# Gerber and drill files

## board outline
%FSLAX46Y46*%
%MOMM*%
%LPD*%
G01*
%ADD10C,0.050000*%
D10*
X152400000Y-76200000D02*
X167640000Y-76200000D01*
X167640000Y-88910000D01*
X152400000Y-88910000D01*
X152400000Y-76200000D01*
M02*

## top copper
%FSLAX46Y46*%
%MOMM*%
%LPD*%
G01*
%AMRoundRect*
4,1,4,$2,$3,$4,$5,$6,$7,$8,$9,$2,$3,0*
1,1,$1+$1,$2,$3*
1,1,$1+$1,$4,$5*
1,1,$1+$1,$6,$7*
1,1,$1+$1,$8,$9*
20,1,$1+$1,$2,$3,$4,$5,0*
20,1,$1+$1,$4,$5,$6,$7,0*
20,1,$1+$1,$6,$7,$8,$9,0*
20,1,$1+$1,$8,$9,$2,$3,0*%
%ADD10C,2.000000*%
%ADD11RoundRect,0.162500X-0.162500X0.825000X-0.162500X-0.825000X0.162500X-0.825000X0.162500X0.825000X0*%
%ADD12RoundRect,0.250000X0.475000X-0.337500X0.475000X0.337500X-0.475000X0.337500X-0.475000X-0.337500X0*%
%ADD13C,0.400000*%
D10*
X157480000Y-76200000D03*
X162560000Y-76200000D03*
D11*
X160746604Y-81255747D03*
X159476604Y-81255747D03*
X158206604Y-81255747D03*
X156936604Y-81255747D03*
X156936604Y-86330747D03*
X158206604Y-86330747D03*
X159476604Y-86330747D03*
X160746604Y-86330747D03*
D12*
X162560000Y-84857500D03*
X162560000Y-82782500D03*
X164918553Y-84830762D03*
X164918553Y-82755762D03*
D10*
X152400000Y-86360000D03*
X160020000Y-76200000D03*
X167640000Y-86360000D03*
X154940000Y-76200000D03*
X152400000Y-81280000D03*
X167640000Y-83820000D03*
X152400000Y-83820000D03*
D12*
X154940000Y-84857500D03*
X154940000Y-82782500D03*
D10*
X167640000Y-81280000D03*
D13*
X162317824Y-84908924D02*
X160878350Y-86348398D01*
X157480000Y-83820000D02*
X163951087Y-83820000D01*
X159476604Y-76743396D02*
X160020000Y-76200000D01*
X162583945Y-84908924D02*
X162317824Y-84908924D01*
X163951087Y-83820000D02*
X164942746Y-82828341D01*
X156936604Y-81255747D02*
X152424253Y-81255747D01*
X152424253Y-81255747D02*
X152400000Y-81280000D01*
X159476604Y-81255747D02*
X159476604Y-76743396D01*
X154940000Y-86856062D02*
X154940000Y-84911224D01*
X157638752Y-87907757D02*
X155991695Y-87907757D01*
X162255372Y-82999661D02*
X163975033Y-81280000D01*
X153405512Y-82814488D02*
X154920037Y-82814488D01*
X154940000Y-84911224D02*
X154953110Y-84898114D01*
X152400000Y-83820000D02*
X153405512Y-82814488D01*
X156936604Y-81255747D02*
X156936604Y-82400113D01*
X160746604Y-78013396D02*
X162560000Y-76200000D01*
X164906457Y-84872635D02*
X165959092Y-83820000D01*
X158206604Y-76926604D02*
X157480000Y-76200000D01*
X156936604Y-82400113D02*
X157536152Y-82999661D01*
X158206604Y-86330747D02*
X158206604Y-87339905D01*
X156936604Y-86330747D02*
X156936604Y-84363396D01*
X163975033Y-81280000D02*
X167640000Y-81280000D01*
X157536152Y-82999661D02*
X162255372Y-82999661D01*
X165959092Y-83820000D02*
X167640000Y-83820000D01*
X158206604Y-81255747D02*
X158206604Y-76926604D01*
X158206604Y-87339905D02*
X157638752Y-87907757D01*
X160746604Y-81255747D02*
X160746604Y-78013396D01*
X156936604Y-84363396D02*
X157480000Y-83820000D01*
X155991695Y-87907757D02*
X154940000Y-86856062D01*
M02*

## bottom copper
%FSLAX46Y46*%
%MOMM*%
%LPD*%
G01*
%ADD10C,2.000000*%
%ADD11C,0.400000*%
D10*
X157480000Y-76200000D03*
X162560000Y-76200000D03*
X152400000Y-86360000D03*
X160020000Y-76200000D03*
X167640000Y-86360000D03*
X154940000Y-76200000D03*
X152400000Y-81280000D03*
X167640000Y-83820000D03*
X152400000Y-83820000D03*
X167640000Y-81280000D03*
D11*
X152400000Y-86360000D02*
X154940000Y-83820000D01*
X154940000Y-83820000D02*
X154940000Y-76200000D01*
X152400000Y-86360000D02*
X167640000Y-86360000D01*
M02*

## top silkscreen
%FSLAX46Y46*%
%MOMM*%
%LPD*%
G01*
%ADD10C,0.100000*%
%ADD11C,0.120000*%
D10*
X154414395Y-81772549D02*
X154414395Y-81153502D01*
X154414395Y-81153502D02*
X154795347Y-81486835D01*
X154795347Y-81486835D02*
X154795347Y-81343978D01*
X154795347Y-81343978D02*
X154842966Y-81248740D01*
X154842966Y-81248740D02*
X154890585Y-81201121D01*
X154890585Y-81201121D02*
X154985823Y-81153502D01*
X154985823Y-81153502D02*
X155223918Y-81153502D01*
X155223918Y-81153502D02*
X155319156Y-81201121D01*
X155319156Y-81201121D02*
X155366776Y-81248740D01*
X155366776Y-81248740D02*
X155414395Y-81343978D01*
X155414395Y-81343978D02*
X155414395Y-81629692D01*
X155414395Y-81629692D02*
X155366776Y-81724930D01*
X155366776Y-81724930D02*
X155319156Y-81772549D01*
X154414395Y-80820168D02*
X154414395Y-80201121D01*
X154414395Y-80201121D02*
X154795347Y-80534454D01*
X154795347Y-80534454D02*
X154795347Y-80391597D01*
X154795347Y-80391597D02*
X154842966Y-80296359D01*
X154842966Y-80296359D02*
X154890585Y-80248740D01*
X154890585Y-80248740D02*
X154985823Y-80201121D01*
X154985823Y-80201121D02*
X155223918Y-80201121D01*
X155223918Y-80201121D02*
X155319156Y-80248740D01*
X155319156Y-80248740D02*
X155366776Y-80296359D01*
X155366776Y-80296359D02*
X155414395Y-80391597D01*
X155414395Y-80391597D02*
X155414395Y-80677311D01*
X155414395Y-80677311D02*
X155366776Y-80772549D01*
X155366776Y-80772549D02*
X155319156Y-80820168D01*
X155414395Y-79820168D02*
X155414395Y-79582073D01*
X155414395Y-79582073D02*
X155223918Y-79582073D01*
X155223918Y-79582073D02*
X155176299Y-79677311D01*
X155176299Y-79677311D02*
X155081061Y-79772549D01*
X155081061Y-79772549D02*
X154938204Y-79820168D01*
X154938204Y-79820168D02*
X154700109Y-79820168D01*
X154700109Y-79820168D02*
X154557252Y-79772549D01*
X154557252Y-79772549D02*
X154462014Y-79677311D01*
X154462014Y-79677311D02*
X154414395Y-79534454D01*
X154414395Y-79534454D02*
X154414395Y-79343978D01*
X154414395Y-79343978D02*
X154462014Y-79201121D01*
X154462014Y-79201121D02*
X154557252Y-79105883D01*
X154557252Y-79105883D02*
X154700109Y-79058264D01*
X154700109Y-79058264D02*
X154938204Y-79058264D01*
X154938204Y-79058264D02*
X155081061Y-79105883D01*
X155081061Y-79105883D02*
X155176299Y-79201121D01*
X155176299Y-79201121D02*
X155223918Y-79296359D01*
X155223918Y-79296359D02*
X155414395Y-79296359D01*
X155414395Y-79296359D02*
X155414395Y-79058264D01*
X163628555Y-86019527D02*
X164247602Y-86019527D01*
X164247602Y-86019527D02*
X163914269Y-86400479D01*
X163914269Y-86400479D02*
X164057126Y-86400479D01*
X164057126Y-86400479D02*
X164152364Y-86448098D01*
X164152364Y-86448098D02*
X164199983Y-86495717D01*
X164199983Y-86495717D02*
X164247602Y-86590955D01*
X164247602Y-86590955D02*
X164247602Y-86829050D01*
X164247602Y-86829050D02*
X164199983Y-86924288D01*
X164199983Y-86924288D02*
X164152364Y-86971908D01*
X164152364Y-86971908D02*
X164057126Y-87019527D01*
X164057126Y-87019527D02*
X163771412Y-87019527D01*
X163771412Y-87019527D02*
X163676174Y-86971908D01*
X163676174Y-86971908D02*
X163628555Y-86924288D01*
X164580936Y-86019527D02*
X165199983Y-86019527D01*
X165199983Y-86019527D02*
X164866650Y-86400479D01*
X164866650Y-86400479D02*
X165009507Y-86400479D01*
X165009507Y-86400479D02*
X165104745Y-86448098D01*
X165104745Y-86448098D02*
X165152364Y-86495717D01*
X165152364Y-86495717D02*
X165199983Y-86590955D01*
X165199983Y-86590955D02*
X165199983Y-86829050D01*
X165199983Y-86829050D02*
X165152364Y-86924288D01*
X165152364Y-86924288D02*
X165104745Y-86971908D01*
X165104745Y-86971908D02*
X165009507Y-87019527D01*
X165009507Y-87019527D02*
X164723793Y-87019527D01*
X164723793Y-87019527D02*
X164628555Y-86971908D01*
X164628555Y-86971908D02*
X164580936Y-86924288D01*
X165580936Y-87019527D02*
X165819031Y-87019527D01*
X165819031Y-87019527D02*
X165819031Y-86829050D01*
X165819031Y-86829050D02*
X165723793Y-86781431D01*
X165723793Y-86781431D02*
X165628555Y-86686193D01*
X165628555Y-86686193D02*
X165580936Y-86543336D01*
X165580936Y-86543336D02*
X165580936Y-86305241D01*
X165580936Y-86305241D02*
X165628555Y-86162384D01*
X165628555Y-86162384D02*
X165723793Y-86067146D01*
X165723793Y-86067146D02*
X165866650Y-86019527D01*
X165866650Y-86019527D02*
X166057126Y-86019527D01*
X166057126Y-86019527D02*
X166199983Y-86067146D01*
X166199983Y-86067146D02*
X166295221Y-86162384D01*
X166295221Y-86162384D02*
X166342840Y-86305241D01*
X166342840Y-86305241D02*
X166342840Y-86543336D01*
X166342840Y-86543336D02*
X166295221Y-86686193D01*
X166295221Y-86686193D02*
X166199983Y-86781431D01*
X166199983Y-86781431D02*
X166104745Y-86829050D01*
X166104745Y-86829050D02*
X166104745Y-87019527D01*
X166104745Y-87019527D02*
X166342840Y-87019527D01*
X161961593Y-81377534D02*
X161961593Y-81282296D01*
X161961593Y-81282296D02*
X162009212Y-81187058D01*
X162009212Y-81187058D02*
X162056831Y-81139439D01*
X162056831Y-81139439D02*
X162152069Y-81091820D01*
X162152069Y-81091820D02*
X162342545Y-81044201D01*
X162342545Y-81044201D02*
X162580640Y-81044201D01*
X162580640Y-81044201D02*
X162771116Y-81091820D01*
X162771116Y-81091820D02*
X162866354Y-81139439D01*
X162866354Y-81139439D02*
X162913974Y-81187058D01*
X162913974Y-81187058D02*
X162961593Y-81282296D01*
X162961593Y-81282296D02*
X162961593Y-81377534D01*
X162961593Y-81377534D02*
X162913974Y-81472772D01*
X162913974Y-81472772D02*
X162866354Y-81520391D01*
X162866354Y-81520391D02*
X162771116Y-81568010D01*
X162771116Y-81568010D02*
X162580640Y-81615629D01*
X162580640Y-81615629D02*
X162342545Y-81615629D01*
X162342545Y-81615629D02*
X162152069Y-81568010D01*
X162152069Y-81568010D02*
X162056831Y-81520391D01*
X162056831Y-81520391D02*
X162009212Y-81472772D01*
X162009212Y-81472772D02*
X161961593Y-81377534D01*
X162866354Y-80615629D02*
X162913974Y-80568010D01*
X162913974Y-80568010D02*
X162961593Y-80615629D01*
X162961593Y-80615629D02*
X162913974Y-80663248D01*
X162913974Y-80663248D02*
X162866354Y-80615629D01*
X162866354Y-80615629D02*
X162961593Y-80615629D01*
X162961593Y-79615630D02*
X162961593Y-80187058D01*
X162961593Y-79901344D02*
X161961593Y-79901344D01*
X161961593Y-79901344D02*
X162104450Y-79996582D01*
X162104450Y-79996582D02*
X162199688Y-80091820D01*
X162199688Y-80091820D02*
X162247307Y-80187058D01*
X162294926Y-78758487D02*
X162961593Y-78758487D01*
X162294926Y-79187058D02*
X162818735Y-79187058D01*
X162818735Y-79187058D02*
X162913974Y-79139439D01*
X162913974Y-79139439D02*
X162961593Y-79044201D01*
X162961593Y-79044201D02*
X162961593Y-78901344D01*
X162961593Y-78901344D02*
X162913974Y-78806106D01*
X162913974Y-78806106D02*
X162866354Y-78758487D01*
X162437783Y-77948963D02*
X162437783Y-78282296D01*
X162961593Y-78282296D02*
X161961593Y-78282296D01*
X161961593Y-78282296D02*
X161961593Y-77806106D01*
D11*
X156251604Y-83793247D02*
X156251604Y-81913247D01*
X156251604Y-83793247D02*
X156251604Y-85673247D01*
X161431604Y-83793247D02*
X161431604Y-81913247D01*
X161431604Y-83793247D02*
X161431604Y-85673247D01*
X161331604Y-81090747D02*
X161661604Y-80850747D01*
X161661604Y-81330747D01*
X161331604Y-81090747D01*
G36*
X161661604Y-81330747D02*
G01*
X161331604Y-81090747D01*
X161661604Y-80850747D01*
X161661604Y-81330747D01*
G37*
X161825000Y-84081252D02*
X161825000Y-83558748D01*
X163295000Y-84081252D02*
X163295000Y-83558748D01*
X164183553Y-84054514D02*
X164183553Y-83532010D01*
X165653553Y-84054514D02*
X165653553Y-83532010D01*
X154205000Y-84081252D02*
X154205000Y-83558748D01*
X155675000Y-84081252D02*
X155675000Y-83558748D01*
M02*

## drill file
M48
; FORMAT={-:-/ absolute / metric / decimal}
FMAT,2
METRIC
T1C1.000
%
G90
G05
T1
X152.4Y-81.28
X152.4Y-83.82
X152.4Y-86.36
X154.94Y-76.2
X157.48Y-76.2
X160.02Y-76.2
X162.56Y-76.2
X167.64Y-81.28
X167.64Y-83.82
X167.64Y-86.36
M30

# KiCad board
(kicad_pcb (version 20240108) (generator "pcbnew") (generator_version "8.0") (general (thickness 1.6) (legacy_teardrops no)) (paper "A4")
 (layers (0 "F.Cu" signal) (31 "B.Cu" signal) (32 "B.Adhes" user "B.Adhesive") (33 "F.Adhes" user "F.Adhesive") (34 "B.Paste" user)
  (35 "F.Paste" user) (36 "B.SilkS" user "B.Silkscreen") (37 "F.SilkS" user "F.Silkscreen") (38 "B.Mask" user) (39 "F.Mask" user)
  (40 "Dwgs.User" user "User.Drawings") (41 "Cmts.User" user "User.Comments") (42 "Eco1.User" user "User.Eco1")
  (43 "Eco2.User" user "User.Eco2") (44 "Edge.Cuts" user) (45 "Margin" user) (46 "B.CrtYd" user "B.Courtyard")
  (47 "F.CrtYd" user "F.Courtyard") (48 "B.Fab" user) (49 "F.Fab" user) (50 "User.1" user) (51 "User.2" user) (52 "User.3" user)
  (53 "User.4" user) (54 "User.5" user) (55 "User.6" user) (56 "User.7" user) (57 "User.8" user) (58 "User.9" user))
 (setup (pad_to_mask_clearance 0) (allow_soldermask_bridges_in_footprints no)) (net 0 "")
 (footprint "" (layer "F.Cu") (at 157.48 76.2)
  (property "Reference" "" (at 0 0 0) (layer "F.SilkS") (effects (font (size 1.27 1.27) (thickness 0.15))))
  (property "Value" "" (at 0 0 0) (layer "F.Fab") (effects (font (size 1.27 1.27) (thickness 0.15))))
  (pad "1" thru_hole circle (at 0 0) (size 2 2) (drill 1) (layers "*.Cu" "*.Mask") (remove_unused_layers no)))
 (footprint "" (layer "F.Cu") (at 162.56 76.2)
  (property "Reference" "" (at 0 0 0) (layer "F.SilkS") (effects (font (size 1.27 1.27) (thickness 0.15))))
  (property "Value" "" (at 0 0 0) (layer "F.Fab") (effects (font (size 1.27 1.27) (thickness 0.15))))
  (pad "1" thru_hole circle (at 0 0) (size 2 2) (drill 1) (layers "*.Cu" "*.Mask") (remove_unused_layers no)))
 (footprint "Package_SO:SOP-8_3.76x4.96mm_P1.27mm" (layer "F.Cu") (at 158.841604 83.793247 -90)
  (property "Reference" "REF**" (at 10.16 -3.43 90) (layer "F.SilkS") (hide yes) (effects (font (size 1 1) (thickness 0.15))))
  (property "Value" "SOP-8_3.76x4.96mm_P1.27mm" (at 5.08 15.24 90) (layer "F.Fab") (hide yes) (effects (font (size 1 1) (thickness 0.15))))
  (fp_line (start 0 2.59) (end -1.88 2.59) (stroke (width 0.12) (type solid)) (layer "F.SilkS"))
  (fp_line (start 0 2.59) (end 1.88 2.59) (stroke (width 0.12) (type solid)) (layer "F.SilkS"))
  (fp_line (start 0 -2.59) (end -1.88 -2.59) (stroke (width 0.12) (type solid)) (layer "F.SilkS"))
  (fp_line (start 0 -2.59) (end 1.88 -2.59) (stroke (width 0.12) (type solid)) (layer "F.SilkS"))
  (fp_poly
   (pts (xy -2.7025 -2.49) (xy -2.9425 -2.82) (xy -2.4625 -2.82) (xy -2.7025 -2.49)) (stroke (width 0.12) (type solid)) (fill solid)
   (layer "F.SilkS"))
  (pad "1" smd roundrect (at -2.5375 -1.905 270) (size 1.975 0.65) (layers "F.Cu" "F.Paste" "F.Mask") (roundrect_rratio 0.25))
  (pad "2" smd roundrect (at -2.5375 -0.635 270) (size 1.975 0.65) (layers "F.Cu" "F.Paste" "F.Mask") (roundrect_rratio 0.25))
  (pad "3" smd roundrect (at -2.5375 0.635 270) (size 1.975 0.65) (layers "F.Cu" "F.Paste" "F.Mask") (roundrect_rratio 0.25))
  (pad "4" smd roundrect (at -2.5375 1.905 270) (size 1.975 0.65) (layers "F.Cu" "F.Paste" "F.Mask") (roundrect_rratio 0.25))
  (pad "5" smd roundrect (at 2.5375 1.905 270) (size 1.975 0.65) (layers "F.Cu" "F.Paste" "F.Mask") (roundrect_rratio 0.25))
  (pad "6" smd roundrect (at 2.5375 0.635 270) (size 1.975 0.65) (layers "F.Cu" "F.Paste" "F.Mask") (roundrect_rratio 0.25))
  (pad "7" smd roundrect (at 2.5375 -0.635 270) (size 1.975 0.65) (layers "F.Cu" "F.Paste" "F.Mask") (roundrect_rratio 0.25))
  (pad "8" smd roundrect (at 2.5375 -1.905 270) (size 1.975 0.65) (layers "F.Cu" "F.Paste" "F.Mask") (roundrect_rratio 0.25)))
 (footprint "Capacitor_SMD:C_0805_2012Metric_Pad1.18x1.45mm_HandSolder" (layer "F.Cu") (at 162.56 83.82 90)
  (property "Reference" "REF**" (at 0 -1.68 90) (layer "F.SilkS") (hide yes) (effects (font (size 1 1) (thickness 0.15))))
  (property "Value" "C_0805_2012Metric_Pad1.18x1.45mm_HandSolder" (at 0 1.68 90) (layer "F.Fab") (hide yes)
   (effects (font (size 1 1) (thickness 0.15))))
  (fp_line (start -0.261252 -0.735) (end 0.261252 -0.735) (stroke (width 0.12) (type solid)) (layer "F.SilkS"))
  (fp_line (start -0.261252 0.735) (end 0.261252 0.735) (stroke (width 0.12) (type solid)) (layer "F.SilkS"))
  (pad "1" smd roundrect (at -1.0375 0 90) (size 1.175 1.45) (layers "F.Cu" "F.Paste" "F.Mask") (roundrect_rratio 0.212766))
  (pad "2" smd roundrect (at 1.0375 0 90) (size 1.175 1.45) (layers "F.Cu" "F.Paste" "F.Mask") (roundrect_rratio 0.212766)))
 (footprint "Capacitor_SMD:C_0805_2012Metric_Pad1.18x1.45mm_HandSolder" (layer "F.Cu") (at 164.918553 83.793262 90)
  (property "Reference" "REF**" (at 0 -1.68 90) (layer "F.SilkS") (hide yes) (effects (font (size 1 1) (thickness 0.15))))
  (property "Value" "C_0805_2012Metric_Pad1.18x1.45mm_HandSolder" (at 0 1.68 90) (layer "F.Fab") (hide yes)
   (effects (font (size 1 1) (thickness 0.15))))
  (fp_line (start -0.261252 -0.735) (end 0.261252 -0.735) (stroke (width 0.12) (type solid)) (layer "F.SilkS"))
  (fp_line (start -0.261252 0.735) (end 0.261252 0.735) (stroke (width 0.12) (type solid)) (layer "F.SilkS"))
  (pad "1" smd roundrect (at -1.0375 0 90) (size 1.175 1.45) (layers "F.Cu" "F.Paste" "F.Mask") (roundrect_rratio 0.212766))
  (pad "2" smd roundrect (at 1.0375 0 90) (size 1.175 1.45) (layers "F.Cu" "F.Paste" "F.Mask") (roundrect_rratio 0.212766)))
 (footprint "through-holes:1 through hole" (layer "F.Cu") (at 152.4 86.36)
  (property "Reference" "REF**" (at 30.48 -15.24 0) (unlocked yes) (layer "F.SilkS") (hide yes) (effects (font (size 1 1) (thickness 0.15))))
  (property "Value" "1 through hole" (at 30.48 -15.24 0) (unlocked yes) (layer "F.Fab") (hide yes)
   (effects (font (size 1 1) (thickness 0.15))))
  (pad "1" thru_hole circle (at 0 0) (size 2 2) (drill 1) (layers "*.Cu" "*.Mask") (remove_unused_layers no)))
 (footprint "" (layer "F.Cu") (at 160.02 76.2)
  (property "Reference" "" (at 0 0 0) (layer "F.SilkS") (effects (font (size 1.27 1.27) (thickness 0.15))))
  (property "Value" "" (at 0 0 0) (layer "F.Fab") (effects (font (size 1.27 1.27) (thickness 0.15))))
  (pad "1" thru_hole circle (at 0 0) (size 2 2) (drill 1) (layers "*.Cu" "*.Mask") (remove_unused_layers no)))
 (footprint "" (layer "F.Cu") (at 167.64 86.36)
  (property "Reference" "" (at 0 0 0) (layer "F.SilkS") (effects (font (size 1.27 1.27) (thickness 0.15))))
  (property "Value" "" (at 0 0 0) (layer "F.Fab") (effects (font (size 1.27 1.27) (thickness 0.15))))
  (pad "1" thru_hole circle (at 0 0) (size 2 2) (drill 1) (layers "*.Cu" "*.Mask") (remove_unused_layers no)))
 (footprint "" (layer "F.Cu") (at 154.94 76.2)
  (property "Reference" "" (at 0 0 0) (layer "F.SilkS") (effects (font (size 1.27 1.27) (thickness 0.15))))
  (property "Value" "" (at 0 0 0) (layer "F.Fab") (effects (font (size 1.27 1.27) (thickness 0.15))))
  (pad "1" thru_hole circle (at 0 0) (size 2 2) (drill 1) (layers "*.Cu" "*.Mask") (remove_unused_layers no)))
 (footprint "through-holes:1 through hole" (layer "F.Cu") (at 152.4 81.28)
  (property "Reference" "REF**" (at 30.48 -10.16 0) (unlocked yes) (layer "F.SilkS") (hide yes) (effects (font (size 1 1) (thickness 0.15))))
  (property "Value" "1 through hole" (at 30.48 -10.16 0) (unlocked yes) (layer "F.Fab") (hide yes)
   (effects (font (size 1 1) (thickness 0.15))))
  (pad "1" thru_hole circle (at 0 0) (size 2 2) (drill 1) (layers "*.Cu" "*.Mask") (remove_unused_layers no)))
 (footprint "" (layer "F.Cu") (at 167.64 83.82)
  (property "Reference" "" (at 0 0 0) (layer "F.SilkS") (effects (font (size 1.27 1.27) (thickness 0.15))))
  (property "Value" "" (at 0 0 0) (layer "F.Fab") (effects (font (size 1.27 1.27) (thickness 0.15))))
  (pad "1" thru_hole circle (at 0 0) (size 2 2) (drill 1) (layers "*.Cu" "*.Mask") (remove_unused_layers no)))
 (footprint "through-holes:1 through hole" (layer "F.Cu") (at 152.4 83.82)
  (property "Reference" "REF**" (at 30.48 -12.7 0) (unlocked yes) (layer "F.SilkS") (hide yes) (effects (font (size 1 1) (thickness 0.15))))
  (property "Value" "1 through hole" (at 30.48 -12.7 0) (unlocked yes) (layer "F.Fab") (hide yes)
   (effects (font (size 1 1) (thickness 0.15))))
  (pad "1" thru_hole circle (at 0 0) (size 2 2) (drill 1) (layers "*.Cu" "*.Mask") (remove_unused_layers no)))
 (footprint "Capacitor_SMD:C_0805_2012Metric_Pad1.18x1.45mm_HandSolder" (layer "F.Cu") (at 154.94 83.82 90)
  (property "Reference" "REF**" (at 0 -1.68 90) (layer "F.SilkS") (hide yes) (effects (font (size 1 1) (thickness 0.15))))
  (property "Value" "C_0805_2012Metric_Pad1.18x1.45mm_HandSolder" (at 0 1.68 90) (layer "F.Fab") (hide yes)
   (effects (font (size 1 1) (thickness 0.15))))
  (fp_line (start -0.261252 -0.735) (end 0.261252 -0.735) (stroke (width 0.12) (type solid)) (layer "F.SilkS"))
  (fp_line (start -0.261252 0.735) (end 0.261252 0.735) (stroke (width 0.12) (type solid)) (layer "F.SilkS"))
  (pad "1" smd roundrect (at -1.0375 0 90) (size 1.175 1.45) (layers "F.Cu" "F.Paste" "F.Mask") (roundrect_rratio 0.212766))
  (pad "2" smd roundrect (at 1.0375 0 90) (size 1.175 1.45) (layers "F.Cu" "F.Paste" "F.Mask") (roundrect_rratio 0.212766)))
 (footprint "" (layer "F.Cu") (at 167.64 81.28)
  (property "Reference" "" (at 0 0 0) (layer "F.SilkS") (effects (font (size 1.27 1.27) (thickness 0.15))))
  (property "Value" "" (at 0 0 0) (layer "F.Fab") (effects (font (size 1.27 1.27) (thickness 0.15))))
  (pad "1" thru_hole circle (at 0 0) (size 2 2) (drill 1) (layers "*.Cu" "*.Mask") (remove_unused_layers no)))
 (gr_rect (start 152.4 76.2) (end 167.64 88.91) (stroke (width 0.05) (type default)) (fill none) (layer "Edge.Cuts"))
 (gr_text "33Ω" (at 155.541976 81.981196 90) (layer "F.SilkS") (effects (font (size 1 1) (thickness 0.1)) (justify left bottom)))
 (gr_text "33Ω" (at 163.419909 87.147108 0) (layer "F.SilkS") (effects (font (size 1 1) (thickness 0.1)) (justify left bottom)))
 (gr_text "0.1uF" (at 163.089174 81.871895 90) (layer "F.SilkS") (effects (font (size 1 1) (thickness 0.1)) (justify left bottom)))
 (segment (start 162.317824 84.908924) (end 160.87835 86.348398) (width 0.4) (layer "F.Cu") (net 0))
 (segment (start 157.48 83.82) (end 163.951087 83.82) (width 0.4) (layer "F.Cu") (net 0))
 (segment (start 159.476604 76.743396) (end 160.02 76.2) (width 0.4) (layer "F.Cu") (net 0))
 (segment (start 162.583945 84.908924) (end 162.317824 84.908924) (width 0.4) (layer "F.Cu") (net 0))
 (segment (start 163.951087 83.82) (end 164.942746 82.828341) (width 0.4) (layer "F.Cu") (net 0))
 (segment (start 156.936604 81.255747) (end 152.424253 81.255747) (width 0.4) (layer "F.Cu") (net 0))
 (segment (start 152.424253 81.255747) (end 152.4 81.28) (width 0.4) (layer "F.Cu") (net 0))
 (segment (start 159.476604 81.255747) (end 159.476604 76.743396) (width 0.4) (layer "F.Cu") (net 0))
 (segment (start 154.94 86.856062) (end 154.94 84.911224) (width 0.4) (layer "F.Cu") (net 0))
 (segment (start 157.638752 87.907757) (end 155.991695 87.907757) (width 0.4) (layer "F.Cu") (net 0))
 (segment (start 162.255372 82.999661) (end 163.975033 81.28) (width 0.4) (layer "F.Cu") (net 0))
 (segment (start 153.405512 82.814488) (end 154.920037 82.814488) (width 0.4) (layer "F.Cu") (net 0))
 (segment (start 154.94 84.911224) (end 154.95311 84.898114) (width 0.4) (layer "F.Cu") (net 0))
 (segment (start 152.4 83.82) (end 153.405512 82.814488) (width 0.4) (layer "F.Cu") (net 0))
 (segment (start 156.936604 81.255747) (end 156.936604 82.400113) (width 0.4) (layer "F.Cu") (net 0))
 (segment (start 160.746604 78.013396) (end 162.56 76.2) (width 0.4) (layer "F.Cu") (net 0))
 (segment (start 164.906457 84.872635) (end 165.959092 83.82) (width 0.4) (layer "F.Cu") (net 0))
 (segment (start 158.206604 76.926604) (end 157.48 76.2) (width 0.4) (layer "F.Cu") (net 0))
 (segment (start 156.936604 82.400113) (end 157.536152 82.999661) (width 0.4) (layer "F.Cu") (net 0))
 (segment (start 158.206604 86.330747) (end 158.206604 87.339905) (width 0.4) (layer "F.Cu") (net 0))
 (segment (start 156.936604 86.330747) (end 156.936604 84.363396) (width 0.4) (layer "F.Cu") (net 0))
 (segment (start 163.975033 81.28) (end 167.64 81.28) (width 0.4) (layer "F.Cu") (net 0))
 (segment (start 157.536152 82.999661) (end 162.255372 82.999661) (width 0.4) (layer "F.Cu") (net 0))
 (segment (start 165.959092 83.82) (end 167.64 83.82) (width 0.4) (layer "F.Cu") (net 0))
 (segment (start 158.206604 81.255747) (end 158.206604 76.926604) (width 0.4) (layer "F.Cu") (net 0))
 (segment (start 158.206604 87.339905) (end 157.638752 87.907757) (width 0.4) (layer "F.Cu") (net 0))
 (segment (start 160.746604 81.255747) (end 160.746604 78.013396) (width 0.4) (layer "F.Cu") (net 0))
 (segment (start 156.936604 84.363396) (end 157.48 83.82) (width 0.4) (layer "F.Cu") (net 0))
 (segment (start 155.991695 87.907757) (end 154.94 86.856062) (width 0.4) (layer "F.Cu") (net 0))
 (segment (start 152.4 86.36) (end 154.94 83.82) (width 0.4) (layer "B.Cu") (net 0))
 (segment (start 154.94 83.82) (end 154.94 76.2) (width 0.4) (layer "B.Cu") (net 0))
 (segment (start 152.4 86.36) (end 167.64 86.36) (width 0.4) (layer "B.Cu") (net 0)))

